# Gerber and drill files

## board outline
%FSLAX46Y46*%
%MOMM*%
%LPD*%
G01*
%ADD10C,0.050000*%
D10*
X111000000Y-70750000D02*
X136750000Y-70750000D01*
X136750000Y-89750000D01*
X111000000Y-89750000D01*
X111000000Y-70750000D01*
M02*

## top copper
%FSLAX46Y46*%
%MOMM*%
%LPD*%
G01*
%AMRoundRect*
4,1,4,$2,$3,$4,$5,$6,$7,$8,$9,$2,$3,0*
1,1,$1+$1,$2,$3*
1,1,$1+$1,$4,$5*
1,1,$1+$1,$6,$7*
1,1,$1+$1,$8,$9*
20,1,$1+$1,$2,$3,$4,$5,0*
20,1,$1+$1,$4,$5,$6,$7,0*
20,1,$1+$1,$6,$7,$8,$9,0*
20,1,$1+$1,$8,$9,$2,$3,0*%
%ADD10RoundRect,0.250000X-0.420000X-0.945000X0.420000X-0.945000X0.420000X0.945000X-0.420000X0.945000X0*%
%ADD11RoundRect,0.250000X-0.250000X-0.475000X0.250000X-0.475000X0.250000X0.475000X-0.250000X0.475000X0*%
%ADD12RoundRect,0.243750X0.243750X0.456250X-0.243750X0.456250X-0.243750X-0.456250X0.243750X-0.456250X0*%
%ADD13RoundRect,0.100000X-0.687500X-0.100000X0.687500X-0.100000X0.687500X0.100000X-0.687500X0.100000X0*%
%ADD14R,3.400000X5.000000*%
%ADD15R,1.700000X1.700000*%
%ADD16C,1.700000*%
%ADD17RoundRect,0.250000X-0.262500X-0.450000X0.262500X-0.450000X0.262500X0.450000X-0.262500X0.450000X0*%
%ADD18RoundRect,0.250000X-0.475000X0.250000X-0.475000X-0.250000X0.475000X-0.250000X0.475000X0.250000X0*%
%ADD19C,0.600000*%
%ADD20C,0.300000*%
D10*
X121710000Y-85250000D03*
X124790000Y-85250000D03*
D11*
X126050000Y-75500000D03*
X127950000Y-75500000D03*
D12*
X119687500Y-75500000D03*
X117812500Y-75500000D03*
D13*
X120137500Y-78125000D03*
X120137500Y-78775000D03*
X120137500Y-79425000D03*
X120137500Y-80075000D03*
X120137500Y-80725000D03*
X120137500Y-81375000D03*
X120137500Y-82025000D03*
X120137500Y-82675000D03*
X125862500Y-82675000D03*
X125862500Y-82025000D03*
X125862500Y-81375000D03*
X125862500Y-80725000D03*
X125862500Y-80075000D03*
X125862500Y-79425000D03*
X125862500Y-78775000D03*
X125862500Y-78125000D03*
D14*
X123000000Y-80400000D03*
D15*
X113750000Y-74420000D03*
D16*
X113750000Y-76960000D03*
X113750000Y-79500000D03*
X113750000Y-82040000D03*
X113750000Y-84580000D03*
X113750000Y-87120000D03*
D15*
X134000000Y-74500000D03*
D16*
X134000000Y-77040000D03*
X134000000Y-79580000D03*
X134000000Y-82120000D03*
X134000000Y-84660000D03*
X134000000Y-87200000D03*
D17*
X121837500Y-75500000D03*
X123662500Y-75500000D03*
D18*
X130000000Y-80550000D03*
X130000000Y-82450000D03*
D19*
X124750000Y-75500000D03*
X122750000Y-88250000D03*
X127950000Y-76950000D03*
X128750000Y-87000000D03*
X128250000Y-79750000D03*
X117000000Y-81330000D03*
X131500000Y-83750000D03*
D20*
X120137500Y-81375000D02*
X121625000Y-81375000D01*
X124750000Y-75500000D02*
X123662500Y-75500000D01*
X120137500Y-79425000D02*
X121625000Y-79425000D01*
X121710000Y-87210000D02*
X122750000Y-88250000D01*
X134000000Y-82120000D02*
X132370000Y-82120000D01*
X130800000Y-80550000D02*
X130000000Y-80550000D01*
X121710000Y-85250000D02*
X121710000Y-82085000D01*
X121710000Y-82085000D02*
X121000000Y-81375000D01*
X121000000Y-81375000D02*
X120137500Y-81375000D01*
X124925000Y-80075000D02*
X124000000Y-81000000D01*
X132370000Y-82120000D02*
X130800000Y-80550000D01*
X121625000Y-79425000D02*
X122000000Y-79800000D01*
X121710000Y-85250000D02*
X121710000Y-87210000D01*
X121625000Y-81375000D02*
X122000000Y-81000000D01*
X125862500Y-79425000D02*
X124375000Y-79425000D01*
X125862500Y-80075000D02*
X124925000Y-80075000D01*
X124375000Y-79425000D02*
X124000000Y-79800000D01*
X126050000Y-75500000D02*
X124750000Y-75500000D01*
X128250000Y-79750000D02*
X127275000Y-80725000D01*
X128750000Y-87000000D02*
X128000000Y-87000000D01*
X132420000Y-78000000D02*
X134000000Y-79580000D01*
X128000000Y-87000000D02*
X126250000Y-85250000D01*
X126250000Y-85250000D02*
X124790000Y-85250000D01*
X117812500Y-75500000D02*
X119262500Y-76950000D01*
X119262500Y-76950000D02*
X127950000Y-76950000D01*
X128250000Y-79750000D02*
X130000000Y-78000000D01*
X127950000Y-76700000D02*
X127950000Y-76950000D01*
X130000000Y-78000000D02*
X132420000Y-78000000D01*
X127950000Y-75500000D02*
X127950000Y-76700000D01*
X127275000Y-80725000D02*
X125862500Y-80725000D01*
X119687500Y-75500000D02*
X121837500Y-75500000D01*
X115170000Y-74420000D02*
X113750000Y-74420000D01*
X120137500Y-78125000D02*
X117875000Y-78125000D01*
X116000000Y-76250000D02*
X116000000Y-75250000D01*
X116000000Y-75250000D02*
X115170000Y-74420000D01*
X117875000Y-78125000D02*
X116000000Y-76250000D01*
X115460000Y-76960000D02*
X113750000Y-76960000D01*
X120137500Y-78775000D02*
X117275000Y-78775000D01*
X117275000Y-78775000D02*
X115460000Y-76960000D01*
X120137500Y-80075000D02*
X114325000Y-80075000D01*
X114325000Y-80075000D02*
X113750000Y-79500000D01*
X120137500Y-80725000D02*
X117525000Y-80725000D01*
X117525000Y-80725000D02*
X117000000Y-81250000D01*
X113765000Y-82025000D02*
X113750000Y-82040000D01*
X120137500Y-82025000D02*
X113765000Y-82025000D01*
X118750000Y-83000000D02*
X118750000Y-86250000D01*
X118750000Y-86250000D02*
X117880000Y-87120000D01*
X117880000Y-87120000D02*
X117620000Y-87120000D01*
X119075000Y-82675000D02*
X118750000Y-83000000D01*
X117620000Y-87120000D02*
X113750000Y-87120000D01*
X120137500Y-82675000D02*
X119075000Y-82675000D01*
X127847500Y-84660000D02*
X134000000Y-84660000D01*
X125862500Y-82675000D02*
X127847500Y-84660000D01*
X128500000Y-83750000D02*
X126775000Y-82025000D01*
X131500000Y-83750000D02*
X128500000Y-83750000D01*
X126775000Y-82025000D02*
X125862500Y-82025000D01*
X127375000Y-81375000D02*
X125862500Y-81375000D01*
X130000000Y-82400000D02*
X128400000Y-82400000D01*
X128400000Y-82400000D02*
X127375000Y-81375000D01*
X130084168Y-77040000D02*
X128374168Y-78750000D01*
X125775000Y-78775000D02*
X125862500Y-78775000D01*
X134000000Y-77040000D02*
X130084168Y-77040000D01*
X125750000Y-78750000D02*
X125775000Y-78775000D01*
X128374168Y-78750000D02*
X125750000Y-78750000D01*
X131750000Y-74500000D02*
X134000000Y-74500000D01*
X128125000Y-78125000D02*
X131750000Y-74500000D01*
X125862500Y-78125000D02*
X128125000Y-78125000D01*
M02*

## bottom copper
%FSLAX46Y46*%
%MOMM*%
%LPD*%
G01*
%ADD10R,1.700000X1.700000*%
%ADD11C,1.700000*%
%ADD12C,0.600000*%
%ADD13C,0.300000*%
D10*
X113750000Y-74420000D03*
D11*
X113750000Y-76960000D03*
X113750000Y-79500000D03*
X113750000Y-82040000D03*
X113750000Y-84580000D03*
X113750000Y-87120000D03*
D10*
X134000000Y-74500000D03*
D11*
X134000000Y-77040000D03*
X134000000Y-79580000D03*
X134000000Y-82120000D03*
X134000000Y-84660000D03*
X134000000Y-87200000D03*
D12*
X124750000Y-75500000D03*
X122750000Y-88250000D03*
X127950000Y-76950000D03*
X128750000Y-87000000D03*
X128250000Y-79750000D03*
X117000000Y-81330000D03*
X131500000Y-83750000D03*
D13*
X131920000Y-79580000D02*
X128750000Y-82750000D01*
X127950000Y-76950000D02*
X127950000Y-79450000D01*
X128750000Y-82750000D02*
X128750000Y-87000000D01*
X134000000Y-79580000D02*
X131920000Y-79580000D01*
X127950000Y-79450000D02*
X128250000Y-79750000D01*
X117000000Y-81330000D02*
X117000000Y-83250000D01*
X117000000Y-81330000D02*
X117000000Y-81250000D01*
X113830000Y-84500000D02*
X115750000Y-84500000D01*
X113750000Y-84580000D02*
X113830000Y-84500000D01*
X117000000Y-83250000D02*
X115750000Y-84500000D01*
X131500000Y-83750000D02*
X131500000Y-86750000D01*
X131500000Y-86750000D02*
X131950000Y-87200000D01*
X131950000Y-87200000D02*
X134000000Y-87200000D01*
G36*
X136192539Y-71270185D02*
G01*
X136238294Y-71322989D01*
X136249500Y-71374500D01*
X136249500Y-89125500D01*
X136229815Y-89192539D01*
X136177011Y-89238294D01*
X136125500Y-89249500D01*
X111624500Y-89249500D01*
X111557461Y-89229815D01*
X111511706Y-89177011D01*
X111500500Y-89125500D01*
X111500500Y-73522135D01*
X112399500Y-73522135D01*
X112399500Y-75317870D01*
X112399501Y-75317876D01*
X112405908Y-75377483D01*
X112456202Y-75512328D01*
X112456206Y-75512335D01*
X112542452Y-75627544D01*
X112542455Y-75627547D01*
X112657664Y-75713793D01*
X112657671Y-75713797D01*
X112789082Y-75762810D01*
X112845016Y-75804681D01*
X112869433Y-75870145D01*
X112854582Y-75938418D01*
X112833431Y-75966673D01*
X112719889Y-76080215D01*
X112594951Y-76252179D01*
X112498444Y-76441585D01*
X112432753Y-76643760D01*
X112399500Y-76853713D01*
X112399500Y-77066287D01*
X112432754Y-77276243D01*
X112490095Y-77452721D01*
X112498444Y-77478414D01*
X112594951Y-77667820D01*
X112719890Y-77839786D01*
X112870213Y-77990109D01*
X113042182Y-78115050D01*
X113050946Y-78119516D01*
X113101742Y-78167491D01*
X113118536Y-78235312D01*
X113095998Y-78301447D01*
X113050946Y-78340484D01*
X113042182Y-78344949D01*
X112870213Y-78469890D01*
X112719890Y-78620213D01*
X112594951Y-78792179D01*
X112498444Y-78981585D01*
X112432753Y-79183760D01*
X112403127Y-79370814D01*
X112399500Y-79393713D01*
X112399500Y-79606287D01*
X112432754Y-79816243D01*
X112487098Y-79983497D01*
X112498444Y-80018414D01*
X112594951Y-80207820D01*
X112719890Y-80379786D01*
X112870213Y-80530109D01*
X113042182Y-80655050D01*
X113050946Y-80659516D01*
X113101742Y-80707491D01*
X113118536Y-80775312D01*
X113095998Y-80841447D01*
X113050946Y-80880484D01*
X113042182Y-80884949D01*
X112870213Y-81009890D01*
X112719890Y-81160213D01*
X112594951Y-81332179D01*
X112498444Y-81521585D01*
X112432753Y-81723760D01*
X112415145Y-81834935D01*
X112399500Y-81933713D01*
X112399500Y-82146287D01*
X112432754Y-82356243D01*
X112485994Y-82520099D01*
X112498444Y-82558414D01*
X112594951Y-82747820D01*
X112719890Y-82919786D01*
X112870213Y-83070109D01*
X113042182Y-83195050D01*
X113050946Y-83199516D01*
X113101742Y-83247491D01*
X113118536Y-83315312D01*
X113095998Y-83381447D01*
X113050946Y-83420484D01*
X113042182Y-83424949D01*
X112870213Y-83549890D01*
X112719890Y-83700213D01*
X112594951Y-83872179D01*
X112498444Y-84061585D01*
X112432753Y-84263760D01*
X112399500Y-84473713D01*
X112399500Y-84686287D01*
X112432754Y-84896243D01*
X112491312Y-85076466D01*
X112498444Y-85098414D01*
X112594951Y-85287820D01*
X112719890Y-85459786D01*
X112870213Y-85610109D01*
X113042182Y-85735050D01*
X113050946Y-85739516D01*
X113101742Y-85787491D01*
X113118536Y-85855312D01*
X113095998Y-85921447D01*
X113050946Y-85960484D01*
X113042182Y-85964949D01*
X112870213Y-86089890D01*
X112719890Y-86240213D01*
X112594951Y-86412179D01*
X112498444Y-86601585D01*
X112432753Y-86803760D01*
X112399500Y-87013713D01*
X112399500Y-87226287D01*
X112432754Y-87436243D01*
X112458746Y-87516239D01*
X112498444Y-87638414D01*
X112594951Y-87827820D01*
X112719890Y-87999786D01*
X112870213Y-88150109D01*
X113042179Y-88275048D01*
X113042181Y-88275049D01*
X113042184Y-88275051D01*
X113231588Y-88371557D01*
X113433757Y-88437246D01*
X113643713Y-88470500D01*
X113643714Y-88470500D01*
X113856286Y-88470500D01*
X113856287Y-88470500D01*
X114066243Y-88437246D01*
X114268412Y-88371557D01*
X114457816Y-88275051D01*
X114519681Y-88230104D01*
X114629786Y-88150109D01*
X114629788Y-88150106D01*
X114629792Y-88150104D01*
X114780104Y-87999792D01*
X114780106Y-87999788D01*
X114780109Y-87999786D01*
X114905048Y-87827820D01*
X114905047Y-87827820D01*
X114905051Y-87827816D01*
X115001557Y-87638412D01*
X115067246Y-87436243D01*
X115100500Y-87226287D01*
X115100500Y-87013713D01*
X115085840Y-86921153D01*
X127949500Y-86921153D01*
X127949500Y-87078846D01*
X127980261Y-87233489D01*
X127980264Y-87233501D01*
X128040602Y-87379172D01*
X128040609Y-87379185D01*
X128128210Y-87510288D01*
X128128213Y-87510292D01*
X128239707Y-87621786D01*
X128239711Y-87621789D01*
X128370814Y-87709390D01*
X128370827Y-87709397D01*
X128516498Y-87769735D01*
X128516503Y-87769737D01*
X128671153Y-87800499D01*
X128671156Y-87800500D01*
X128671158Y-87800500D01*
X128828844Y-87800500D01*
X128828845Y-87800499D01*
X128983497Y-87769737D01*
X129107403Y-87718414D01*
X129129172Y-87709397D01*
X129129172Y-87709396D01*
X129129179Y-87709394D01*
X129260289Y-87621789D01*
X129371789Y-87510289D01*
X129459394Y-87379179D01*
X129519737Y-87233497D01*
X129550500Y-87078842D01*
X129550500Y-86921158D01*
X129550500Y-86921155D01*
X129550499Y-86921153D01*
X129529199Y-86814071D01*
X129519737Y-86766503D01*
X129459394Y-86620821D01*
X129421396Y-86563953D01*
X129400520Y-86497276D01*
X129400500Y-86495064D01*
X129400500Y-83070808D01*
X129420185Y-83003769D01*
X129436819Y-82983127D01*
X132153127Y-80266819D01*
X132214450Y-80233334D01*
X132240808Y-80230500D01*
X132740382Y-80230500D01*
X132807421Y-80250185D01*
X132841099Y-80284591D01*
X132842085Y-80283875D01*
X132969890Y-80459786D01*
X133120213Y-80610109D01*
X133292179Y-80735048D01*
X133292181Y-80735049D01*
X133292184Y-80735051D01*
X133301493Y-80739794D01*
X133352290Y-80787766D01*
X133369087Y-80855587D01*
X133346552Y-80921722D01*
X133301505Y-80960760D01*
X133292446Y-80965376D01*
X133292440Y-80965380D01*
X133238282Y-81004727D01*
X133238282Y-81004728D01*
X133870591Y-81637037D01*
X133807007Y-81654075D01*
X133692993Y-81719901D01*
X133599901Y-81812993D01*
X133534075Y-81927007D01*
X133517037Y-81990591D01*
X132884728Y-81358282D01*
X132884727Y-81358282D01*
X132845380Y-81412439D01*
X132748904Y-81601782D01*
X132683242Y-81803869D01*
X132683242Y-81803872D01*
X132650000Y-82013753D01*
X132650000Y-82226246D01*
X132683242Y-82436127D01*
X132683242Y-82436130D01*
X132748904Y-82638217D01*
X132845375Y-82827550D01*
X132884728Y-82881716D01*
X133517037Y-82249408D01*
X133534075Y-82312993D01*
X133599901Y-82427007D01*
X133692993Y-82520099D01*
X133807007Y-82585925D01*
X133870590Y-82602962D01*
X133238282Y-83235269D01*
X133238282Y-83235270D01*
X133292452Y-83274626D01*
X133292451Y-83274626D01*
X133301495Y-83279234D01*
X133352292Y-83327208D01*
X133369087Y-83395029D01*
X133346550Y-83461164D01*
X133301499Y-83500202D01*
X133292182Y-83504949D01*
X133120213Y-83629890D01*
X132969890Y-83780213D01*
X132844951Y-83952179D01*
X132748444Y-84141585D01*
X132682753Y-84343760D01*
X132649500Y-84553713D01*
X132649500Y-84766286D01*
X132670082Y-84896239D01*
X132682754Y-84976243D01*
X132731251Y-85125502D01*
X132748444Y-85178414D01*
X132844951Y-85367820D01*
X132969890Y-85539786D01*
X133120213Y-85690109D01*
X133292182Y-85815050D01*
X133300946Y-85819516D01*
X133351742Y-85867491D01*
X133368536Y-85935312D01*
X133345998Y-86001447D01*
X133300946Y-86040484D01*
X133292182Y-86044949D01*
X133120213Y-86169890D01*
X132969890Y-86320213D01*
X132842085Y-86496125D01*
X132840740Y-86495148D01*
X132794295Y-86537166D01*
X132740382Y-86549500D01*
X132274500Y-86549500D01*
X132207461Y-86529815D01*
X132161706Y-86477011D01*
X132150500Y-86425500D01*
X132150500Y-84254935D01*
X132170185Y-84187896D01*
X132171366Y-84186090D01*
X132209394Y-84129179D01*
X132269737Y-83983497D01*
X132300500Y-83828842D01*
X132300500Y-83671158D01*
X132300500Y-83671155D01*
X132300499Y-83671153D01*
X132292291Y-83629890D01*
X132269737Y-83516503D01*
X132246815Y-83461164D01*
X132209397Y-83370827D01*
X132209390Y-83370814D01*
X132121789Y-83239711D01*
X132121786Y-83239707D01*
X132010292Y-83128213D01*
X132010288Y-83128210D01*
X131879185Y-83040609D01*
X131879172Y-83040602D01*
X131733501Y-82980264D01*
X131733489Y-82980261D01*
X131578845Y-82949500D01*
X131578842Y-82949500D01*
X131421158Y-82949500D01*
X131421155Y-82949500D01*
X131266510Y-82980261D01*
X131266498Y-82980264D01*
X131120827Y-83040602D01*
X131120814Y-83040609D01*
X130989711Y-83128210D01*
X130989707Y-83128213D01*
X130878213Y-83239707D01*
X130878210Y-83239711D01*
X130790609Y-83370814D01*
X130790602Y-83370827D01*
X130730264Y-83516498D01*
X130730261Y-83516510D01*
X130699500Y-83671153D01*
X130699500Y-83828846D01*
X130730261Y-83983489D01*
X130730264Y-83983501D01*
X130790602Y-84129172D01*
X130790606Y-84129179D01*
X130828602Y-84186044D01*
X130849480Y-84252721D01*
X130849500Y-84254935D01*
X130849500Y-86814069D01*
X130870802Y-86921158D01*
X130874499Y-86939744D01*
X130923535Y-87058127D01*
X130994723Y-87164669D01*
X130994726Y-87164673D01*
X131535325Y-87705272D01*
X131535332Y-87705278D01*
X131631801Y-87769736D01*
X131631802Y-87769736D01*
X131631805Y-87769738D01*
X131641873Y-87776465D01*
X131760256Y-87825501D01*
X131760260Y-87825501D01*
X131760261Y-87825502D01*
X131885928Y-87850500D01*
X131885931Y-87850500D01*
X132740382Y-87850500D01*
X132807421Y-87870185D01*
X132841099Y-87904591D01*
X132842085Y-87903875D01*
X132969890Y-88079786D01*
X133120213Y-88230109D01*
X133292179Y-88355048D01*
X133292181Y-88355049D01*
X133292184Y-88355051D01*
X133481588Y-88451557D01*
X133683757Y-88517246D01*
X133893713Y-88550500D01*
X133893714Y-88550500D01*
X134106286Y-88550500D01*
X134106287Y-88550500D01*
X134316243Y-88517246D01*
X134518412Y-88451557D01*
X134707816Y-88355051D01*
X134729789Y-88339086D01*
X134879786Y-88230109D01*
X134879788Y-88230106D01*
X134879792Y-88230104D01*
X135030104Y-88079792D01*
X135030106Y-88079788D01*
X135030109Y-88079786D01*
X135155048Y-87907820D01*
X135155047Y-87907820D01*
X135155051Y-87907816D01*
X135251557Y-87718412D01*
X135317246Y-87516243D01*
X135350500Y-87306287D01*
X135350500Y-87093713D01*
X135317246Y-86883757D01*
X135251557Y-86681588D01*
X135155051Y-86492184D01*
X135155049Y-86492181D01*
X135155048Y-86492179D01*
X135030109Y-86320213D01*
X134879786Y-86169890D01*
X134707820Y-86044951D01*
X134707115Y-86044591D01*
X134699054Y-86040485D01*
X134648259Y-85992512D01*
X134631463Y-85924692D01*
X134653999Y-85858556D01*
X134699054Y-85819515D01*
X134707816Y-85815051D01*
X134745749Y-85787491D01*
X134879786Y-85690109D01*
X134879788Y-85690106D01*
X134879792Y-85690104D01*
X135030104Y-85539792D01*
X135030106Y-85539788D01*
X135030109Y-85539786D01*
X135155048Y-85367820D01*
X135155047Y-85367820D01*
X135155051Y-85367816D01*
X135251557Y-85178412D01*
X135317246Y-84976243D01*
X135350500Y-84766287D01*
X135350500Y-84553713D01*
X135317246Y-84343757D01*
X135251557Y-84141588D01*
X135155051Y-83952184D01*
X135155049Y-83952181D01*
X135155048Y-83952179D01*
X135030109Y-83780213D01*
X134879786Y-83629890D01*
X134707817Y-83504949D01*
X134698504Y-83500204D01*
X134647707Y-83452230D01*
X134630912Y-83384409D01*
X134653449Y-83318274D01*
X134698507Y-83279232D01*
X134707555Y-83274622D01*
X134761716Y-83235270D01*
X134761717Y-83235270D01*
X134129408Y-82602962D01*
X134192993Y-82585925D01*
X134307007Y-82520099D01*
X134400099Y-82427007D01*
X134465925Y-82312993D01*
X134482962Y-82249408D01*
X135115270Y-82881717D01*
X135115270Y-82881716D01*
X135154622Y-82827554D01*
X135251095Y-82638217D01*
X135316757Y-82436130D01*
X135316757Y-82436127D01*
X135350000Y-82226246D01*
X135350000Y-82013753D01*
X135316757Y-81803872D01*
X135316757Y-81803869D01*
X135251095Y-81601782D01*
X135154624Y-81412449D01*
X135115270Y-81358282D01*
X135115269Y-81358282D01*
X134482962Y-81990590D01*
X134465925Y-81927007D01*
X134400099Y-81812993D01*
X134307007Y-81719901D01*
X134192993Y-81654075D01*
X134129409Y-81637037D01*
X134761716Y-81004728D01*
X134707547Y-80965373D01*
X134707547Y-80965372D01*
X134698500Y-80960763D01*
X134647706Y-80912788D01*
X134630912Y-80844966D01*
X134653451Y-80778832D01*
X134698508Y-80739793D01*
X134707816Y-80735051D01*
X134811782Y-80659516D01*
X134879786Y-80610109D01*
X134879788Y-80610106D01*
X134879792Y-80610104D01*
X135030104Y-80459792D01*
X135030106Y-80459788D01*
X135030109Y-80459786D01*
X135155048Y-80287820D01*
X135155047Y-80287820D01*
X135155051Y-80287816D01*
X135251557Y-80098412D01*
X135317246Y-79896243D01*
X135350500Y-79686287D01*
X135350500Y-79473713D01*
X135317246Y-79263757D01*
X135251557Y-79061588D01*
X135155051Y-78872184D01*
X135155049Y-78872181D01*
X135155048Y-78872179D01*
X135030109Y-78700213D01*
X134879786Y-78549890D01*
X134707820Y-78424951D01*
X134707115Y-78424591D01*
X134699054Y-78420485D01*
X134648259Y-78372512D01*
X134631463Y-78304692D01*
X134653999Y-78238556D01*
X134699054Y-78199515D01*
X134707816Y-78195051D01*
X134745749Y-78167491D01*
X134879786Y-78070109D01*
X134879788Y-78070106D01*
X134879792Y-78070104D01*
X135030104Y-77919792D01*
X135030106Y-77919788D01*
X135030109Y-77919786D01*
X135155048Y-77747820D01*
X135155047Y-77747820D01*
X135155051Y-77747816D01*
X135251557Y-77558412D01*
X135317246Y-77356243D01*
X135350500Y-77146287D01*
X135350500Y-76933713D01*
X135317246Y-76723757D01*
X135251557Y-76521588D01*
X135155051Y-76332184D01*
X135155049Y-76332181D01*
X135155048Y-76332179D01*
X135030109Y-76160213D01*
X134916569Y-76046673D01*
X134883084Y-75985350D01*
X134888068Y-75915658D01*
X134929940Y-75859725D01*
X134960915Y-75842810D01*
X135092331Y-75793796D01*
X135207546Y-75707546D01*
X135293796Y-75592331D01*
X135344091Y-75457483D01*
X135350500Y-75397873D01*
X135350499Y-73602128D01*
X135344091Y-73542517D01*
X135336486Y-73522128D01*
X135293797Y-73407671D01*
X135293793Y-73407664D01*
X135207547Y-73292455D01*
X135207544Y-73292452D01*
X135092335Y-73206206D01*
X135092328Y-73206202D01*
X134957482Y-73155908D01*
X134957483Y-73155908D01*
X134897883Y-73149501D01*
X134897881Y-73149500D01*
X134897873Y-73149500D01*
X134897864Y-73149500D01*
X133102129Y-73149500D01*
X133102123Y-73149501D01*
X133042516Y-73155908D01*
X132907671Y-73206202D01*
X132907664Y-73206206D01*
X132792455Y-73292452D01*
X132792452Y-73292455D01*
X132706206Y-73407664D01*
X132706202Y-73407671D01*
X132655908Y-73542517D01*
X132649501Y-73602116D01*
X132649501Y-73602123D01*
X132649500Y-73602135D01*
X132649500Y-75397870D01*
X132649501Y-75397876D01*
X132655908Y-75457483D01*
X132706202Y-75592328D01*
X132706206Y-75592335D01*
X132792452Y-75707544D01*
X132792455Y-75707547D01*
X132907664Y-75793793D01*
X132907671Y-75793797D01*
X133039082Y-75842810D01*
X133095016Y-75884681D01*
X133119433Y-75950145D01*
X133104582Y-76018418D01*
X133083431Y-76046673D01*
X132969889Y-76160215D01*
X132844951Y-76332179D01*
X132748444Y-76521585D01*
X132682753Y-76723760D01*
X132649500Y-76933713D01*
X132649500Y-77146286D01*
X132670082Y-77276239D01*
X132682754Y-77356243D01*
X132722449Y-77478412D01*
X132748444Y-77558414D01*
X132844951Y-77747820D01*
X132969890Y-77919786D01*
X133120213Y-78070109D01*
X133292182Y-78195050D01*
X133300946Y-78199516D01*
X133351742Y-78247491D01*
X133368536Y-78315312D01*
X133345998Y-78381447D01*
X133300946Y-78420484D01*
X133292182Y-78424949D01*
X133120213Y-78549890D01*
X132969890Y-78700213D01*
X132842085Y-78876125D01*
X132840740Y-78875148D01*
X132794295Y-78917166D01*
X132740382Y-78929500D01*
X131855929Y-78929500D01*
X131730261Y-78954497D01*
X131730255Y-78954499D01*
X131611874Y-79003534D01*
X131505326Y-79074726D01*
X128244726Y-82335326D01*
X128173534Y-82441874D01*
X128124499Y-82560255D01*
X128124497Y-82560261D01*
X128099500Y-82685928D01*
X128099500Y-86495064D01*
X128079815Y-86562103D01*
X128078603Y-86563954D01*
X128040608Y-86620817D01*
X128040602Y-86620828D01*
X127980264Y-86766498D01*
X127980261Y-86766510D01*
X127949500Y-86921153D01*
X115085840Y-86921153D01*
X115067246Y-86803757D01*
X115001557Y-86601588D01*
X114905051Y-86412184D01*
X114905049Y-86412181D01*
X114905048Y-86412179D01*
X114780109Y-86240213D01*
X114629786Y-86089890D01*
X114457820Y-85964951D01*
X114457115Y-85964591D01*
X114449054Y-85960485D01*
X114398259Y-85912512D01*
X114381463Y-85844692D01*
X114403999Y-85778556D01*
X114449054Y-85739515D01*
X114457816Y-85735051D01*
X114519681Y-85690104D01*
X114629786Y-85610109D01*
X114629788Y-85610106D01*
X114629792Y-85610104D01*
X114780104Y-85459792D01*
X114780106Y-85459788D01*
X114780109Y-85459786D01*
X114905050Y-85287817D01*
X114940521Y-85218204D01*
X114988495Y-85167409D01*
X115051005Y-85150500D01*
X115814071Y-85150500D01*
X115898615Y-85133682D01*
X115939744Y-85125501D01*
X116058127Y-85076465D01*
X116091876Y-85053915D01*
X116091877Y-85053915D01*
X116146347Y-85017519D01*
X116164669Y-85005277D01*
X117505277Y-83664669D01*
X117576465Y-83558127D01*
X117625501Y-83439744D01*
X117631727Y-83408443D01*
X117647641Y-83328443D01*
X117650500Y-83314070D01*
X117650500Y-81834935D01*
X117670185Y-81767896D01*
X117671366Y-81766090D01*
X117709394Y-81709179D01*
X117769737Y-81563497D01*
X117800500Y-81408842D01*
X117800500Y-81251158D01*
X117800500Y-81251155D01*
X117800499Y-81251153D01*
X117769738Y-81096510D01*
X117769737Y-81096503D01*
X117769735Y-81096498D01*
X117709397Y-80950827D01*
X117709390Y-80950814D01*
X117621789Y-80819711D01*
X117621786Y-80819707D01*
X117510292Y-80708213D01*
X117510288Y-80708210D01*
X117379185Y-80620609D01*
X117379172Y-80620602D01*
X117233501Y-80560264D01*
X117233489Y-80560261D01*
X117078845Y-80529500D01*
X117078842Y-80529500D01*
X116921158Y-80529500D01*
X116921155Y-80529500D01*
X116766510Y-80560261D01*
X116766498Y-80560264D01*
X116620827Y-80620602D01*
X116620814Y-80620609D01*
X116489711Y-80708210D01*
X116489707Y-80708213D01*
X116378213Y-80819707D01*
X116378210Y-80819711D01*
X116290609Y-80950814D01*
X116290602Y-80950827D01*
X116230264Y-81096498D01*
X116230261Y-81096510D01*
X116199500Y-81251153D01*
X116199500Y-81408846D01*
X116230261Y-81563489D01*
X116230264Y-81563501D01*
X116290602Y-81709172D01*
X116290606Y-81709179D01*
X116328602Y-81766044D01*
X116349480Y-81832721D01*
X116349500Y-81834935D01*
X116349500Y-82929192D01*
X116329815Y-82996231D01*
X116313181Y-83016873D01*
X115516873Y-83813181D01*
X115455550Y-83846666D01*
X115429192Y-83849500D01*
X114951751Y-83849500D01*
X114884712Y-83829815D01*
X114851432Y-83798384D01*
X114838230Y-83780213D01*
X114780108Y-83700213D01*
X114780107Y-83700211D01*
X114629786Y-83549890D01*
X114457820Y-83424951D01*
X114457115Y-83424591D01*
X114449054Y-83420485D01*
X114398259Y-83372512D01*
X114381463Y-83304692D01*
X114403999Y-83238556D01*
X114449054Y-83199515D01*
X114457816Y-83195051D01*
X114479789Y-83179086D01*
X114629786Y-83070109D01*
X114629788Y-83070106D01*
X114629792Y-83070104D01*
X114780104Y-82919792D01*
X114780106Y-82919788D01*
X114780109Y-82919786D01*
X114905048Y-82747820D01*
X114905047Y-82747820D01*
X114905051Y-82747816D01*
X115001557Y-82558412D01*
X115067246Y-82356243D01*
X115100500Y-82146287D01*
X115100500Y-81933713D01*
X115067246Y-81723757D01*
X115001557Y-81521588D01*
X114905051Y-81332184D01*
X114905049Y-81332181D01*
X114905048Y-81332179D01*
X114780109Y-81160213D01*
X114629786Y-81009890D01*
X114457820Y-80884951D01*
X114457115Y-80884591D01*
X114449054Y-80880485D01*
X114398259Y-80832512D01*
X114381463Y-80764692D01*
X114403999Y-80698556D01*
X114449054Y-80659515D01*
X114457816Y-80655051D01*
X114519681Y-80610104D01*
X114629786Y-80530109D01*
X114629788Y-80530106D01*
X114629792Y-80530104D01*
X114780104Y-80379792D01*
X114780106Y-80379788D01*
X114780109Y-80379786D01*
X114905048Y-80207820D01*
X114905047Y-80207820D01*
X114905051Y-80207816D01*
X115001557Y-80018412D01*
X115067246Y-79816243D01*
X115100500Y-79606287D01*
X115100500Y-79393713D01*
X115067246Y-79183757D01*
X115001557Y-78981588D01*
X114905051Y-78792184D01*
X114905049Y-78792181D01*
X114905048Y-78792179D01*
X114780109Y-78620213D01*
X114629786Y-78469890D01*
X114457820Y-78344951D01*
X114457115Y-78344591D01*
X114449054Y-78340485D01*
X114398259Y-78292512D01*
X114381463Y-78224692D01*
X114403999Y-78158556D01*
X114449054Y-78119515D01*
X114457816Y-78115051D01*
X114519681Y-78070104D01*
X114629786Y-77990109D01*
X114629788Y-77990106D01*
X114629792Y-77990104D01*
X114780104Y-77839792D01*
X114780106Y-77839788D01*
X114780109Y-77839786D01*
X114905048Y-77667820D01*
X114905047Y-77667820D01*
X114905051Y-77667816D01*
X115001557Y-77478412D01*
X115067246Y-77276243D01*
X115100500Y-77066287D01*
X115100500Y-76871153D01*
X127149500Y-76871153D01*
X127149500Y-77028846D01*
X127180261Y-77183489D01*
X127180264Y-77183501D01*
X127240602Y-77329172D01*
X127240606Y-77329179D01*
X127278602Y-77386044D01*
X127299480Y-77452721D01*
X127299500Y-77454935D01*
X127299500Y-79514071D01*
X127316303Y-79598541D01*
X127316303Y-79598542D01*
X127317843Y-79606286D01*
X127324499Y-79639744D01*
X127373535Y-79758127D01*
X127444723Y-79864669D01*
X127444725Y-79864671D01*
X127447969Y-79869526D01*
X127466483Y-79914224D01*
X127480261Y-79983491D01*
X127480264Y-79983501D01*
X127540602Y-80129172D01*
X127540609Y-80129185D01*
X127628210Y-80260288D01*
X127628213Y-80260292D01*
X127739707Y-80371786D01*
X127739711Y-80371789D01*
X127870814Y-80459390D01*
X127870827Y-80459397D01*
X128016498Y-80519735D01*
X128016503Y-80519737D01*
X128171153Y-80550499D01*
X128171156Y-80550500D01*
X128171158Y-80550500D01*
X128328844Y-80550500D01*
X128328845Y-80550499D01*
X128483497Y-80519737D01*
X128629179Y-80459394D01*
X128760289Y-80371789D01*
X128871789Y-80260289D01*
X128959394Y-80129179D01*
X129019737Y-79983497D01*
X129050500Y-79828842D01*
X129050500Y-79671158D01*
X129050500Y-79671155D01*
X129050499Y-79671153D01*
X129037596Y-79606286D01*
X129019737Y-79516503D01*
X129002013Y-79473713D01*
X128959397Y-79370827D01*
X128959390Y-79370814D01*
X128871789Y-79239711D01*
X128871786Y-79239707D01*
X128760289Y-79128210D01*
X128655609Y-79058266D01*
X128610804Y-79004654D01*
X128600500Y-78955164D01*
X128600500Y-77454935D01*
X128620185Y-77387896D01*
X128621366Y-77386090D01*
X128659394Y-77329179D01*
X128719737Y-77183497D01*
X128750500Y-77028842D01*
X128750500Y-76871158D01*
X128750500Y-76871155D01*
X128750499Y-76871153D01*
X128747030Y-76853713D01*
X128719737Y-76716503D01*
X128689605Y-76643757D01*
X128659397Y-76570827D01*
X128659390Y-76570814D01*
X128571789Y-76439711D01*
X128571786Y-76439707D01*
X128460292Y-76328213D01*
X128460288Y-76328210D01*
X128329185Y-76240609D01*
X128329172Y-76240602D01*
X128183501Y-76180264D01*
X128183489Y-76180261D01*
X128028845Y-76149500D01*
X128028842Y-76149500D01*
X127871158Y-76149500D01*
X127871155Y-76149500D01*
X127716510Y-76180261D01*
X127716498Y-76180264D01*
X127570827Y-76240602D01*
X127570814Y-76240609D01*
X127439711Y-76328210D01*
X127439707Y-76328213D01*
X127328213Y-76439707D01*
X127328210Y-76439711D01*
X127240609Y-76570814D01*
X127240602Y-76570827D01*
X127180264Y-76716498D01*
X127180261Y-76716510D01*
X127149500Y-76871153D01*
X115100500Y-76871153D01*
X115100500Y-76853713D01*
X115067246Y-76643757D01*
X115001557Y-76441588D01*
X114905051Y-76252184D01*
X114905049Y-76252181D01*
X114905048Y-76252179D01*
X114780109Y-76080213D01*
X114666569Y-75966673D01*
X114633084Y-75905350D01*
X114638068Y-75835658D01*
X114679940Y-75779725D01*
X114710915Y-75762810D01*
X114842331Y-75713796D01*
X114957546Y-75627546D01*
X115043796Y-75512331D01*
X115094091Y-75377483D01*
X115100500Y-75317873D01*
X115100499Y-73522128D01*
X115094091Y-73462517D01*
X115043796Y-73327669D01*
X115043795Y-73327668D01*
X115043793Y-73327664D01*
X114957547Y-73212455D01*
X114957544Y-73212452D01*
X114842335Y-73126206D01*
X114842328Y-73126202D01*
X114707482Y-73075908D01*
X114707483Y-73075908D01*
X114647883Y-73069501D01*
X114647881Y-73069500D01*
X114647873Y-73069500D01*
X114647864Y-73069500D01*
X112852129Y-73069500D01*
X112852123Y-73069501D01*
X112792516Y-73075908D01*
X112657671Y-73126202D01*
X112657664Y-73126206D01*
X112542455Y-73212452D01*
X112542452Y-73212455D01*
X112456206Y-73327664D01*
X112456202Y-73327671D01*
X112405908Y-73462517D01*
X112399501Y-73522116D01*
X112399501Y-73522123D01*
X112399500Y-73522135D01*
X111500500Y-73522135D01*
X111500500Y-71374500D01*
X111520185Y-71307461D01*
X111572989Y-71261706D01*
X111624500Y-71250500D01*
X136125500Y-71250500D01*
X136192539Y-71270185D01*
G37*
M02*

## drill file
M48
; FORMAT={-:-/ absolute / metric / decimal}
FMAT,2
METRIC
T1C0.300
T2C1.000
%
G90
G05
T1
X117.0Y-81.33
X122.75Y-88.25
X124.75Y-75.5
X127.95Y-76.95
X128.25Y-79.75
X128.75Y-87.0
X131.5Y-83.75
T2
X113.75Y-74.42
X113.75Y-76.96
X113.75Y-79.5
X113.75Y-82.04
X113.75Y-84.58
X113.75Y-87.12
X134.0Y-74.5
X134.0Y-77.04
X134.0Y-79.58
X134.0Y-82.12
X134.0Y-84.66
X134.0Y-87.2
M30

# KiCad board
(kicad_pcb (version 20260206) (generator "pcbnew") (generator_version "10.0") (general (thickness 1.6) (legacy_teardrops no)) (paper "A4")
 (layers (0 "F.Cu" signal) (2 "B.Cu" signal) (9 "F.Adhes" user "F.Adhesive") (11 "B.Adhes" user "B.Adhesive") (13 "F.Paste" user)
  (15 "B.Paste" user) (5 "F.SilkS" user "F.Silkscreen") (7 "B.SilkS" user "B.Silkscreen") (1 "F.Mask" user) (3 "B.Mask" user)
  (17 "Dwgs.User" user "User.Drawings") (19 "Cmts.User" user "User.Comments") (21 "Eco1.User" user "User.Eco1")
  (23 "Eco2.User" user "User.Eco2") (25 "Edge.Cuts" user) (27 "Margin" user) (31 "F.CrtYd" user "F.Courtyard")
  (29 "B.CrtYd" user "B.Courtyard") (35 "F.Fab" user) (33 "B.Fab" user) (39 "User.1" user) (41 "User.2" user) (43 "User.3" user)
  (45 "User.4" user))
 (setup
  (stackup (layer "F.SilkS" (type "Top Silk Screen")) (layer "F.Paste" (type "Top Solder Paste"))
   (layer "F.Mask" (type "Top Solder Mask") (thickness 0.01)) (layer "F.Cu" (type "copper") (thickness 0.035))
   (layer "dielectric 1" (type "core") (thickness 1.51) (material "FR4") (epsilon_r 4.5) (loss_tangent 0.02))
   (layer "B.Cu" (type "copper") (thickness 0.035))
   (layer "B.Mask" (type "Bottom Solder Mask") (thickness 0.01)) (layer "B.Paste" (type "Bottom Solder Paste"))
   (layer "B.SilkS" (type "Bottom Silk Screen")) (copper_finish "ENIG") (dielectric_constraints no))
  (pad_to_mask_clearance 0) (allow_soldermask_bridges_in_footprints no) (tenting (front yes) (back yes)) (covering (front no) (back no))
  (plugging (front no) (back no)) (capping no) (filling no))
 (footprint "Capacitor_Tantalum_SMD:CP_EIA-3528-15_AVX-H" (layer "F.Cu") (at 123.25 85.25)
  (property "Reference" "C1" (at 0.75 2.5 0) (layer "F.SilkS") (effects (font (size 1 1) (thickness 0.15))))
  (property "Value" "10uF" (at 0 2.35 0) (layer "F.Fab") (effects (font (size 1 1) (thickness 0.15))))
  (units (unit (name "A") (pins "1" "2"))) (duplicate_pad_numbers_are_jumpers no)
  (pad "1" smd roundrect (at -1.54 0) (size 1.34 2.39) (layers "F.Cu" "F.Mask" "F.Paste") (roundrect_rratio 0.186567) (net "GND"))
  (pad "2" smd roundrect (at 1.54 0) (size 1.34 2.39) (layers "F.Cu" "F.Mask" "F.Paste") (roundrect_rratio 0.186567) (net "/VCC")))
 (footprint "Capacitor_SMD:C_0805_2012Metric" (layer "F.Cu") (at 127 75.5)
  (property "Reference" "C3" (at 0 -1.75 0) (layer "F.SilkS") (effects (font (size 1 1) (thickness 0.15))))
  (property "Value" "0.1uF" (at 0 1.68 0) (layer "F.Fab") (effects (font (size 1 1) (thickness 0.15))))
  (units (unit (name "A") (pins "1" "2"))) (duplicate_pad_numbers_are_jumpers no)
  (pad "1" smd roundrect (at -0.95 0) (size 1 1.45) (layers "F.Cu" "F.Mask" "F.Paste") (roundrect_rratio 0.25) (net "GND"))
  (pad "2" smd roundrect (at 0.95 0) (size 1 1.45) (layers "F.Cu" "F.Mask" "F.Paste") (roundrect_rratio 0.25) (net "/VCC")))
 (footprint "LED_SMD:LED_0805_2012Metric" (layer "F.Cu") (at 118.75 75.5 180)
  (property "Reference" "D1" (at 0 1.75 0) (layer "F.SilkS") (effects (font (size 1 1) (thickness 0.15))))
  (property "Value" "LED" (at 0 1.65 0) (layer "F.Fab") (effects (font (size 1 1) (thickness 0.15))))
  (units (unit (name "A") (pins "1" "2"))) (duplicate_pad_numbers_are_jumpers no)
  (pad "1" smd roundrect (at -0.9375 0 180) (size 0.975 1.4) (layers "F.Cu" "F.Mask" "F.Paste") (roundrect_rratio 0.25) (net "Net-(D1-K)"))
  (pad "2" smd roundrect (at 0.9375 0 180) (size 0.975 1.4) (layers "F.Cu" "F.Mask" "F.Paste") (roundrect_rratio 0.25) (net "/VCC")))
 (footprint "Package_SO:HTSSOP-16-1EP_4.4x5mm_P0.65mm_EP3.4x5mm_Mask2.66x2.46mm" (layer "F.Cu") (at 123 80.4)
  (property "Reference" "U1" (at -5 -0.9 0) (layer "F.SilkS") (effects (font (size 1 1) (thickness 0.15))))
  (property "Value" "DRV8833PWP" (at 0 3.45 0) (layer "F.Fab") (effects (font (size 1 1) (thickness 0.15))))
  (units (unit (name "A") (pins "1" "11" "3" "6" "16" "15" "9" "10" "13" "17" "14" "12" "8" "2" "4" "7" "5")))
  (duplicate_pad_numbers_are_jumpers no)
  (pad "" smd roundrect (at 0 -0.615) (size 2.14 0.99) (layers "F.Paste") (roundrect_rratio 0.25))
  (pad "" smd rect (at 0 0) (size 2.66 2.46) (layers "F.Mask"))
  (pad "" smd roundrect (at 0 0.615) (size 2.14 0.99) (layers "F.Paste") (roundrect_rratio 0.25))
  (pad "1" smd roundrect (at -2.8625 -2.275) (size 1.575 0.4) (layers "F.Cu" "F.Mask" "F.Paste") (roundrect_rratio 0.25) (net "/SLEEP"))
  (pad "2" smd roundrect (at -2.8625 -1.625) (size 1.575 0.4) (layers "F.Cu" "F.Mask" "F.Paste") (roundrect_rratio 0.25) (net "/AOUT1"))
  (pad "3" smd roundrect (at -2.8625 -0.975) (size 1.575 0.4) (layers "F.Cu" "F.Mask" "F.Paste") (roundrect_rratio 0.25) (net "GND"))
  (pad "4" smd roundrect (at -2.8625 -0.325) (size 1.575 0.4) (layers "F.Cu" "F.Mask" "F.Paste") (roundrect_rratio 0.25) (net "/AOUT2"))
  (pad "5" smd roundrect (at -2.8625 0.325) (size 1.575 0.4) (layers "F.Cu" "F.Mask" "F.Paste") (roundrect_rratio 0.25) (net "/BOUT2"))
  (pad "6" smd roundrect (at -2.8625 0.975) (size 1.575 0.4) (layers "F.Cu" "F.Mask" "F.Paste") (roundrect_rratio 0.25) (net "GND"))
  (pad "7" smd roundrect (at -2.8625 1.625) (size 1.575 0.4) (layers "F.Cu" "F.Mask" "F.Paste") (roundrect_rratio 0.25) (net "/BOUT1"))
  (pad "8" smd roundrect (at -2.8625 2.275) (size 1.575 0.4) (layers "F.Cu" "F.Mask" "F.Paste") (roundrect_rratio 0.25) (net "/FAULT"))
  (pad "9" smd roundrect (at 2.8625 2.275) (size 1.575 0.4) (layers "F.Cu" "F.Mask" "F.Paste") (roundrect_rratio 0.25) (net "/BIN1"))
  (pad "10" smd roundrect (at 2.8625 1.625) (size 1.575 0.4) (layers "F.Cu" "F.Mask" "F.Paste") (roundrect_rratio 0.25) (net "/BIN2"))
  (pad "11" smd roundrect (at 2.8625 0.975) (size 1.575 0.4) (layers "F.Cu" "F.Mask" "F.Paste") (roundrect_rratio 0.25) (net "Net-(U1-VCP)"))
  (pad "12" smd roundrect (at 2.8625 0.325) (size 1.575 0.4) (layers "F.Cu" "F.Mask" "F.Paste") (roundrect_rratio 0.25) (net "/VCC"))
  (pad "13" smd roundrect (at 2.8625 -0.325) (size 1.575 0.4) (layers "F.Cu" "F.Mask" "F.Paste") (roundrect_rratio 0.25) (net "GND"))
  (pad "14" smd roundrect (at 2.8625 -0.975) (size 1.575 0.4) (layers "F.Cu" "F.Mask" "F.Paste") (roundrect_rratio 0.25) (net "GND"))
  (pad "15" smd roundrect (at 2.8625 -1.625) (size 1.575 0.4) (layers "F.Cu" "F.Mask" "F.Paste") (roundrect_rratio 0.25) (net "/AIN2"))
  (pad "16" smd roundrect (at 2.8625 -2.275) (size 1.575 0.4) (layers "F.Cu" "F.Mask" "F.Paste") (roundrect_rratio 0.25) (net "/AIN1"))
  (pad "17" smd rect (at 0 0) (size 3.4 5) (layers "F.Cu") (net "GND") (zone_connect 2)))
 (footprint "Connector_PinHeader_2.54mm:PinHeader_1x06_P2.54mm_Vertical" (layer "F.Cu") (at 113.75 74.42)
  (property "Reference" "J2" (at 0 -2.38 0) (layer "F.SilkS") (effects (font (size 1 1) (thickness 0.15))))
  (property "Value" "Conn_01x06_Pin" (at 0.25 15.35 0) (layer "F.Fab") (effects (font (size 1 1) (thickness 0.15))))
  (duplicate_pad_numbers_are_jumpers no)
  (pad "1" thru_hole rect (at 0 0) (size 1.7 1.7) (drill 1) (layers "*.Cu" "*.Mask") (remove_unused_layers no) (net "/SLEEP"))
  (pad "2" thru_hole circle (at 0 2.54) (size 1.7 1.7) (drill 1) (layers "*.Cu" "*.Mask") (remove_unused_layers no) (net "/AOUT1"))
  (pad "3" thru_hole circle (at 0 5.08) (size 1.7 1.7) (drill 1) (layers "*.Cu" "*.Mask") (remove_unused_layers no) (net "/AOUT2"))
  (pad "4" thru_hole circle (at 0 7.62) (size 1.7 1.7) (drill 1) (layers "*.Cu" "*.Mask") (remove_unused_layers no) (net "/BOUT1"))
  (pad "5" thru_hole circle (at 0 10.16) (size 1.7 1.7) (drill 1) (layers "*.Cu" "*.Mask") (remove_unused_layers no) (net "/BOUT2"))
  (pad "6" thru_hole circle (at 0 12.7) (size 1.7 1.7) (drill 1) (layers "*.Cu" "*.Mask") (remove_unused_layers no) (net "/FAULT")))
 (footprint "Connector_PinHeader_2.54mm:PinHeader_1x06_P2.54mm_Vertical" (layer "F.Cu") (at 134 74.5)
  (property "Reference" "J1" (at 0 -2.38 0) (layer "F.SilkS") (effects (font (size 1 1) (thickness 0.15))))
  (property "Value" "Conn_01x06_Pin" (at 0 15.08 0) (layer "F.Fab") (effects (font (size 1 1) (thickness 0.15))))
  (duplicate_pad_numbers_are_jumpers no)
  (pad "1" thru_hole rect (at 0 0) (size 1.7 1.7) (drill 1) (layers "*.Cu" "*.Mask") (remove_unused_layers no) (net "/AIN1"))
  (pad "2" thru_hole circle (at 0 2.54) (size 1.7 1.7) (drill 1) (layers "*.Cu" "*.Mask") (remove_unused_layers no) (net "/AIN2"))
  (pad "3" thru_hole circle (at 0 5.08) (size 1.7 1.7) (drill 1) (layers "*.Cu" "*.Mask") (remove_unused_layers no) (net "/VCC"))
  (pad "4" thru_hole circle (at 0 7.62) (size 1.7 1.7) (drill 1) (layers "*.Cu" "*.Mask") (remove_unused_layers no) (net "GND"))
  (pad "5" thru_hole circle (at 0 10.16) (size 1.7 1.7) (drill 1) (layers "*.Cu" "*.Mask") (remove_unused_layers no) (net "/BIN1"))
  (pad "6" thru_hole circle (at 0 12.7) (size 1.7 1.7) (drill 1) (layers "*.Cu" "*.Mask") (remove_unused_layers no) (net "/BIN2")))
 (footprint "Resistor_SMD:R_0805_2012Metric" (layer "F.Cu") (at 122.75 75.5)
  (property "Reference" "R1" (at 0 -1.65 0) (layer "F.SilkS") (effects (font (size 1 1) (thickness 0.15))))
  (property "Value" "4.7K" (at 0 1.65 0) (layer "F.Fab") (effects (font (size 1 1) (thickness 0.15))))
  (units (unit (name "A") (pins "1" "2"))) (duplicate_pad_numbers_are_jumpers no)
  (pad "1" smd roundrect (at -0.9125 0) (size 1.025 1.4) (layers "F.Cu" "F.Mask" "F.Paste") (roundrect_rratio 0.243902) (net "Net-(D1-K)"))
  (pad "2" smd roundrect (at 0.9125 0) (size 1.025 1.4) (layers "F.Cu" "F.Mask" "F.Paste") (roundrect_rratio 0.243902) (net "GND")))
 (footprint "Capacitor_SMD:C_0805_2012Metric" (layer "F.Cu") (at 130 81.5 -90)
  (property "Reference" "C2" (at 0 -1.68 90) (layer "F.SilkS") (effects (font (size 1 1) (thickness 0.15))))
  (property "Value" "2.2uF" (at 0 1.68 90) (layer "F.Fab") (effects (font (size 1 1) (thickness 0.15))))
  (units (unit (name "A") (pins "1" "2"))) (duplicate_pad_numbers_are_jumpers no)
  (pad "1" smd roundrect (at -0.95 0 270) (size 1 1.45) (layers "F.Cu" "F.Mask" "F.Paste") (roundrect_rratio 0.25) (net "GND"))
  (pad "2" smd roundrect (at 0.95 0 270) (size 1 1.45) (layers "F.Cu" "F.Mask" "F.Paste") (roundrect_rratio 0.25) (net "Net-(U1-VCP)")))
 (gr_rect (start 111 70.75) (end 136.75 89.75) (stroke (width 0.05) (type default)) (fill no) (layer "Edge.Cuts"))
 (segment (start 120.1375 81.375) (end 121.625 81.375) (width 0.3) (layer "F.Cu") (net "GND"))
 (segment (start 124.75 75.5) (end 123.6625 75.5) (width 0.3) (layer "F.Cu") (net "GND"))
 (segment (start 120.1375 79.425) (end 121.625 79.425) (width 0.3) (layer "F.Cu") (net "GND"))
 (segment (start 121.71 87.21) (end 122.75 88.25) (width 0.3) (layer "F.Cu") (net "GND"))
 (segment (start 134 82.12) (end 132.37 82.12) (width 0.3) (layer "F.Cu") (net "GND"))
 (segment (start 130.8 80.55) (end 130 80.55) (width 0.3) (layer "F.Cu") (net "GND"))
 (segment (start 121.71 85.25) (end 121.71 82.085) (width 0.3) (layer "F.Cu") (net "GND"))
 (segment (start 121.71 82.085) (end 121 81.375) (width 0.3) (layer "F.Cu") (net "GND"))
 (segment (start 121 81.375) (end 120.1375 81.375) (width 0.3) (layer "F.Cu") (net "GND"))
 (segment (start 124.925 80.075) (end 124 81) (width 0.3) (layer "F.Cu") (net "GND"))
 (segment (start 132.37 82.12) (end 130.8 80.55) (width 0.3) (layer "F.Cu") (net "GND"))
 (segment (start 121.625 79.425) (end 122 79.8) (width 0.3) (layer "F.Cu") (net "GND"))
 (segment (start 121.71 85.25) (end 121.71 87.21) (width 0.3) (layer "F.Cu") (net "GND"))
 (segment (start 121.625 81.375) (end 122 81) (width 0.3) (layer "F.Cu") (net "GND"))
 (segment (start 125.8625 79.425) (end 124.375 79.425) (width 0.3) (layer "F.Cu") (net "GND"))
 (segment (start 125.8625 80.075) (end 124.925 80.075) (width 0.3) (layer "F.Cu") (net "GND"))
 (segment (start 124.375 79.425) (end 124 79.8) (width 0.3) (layer "F.Cu") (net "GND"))
 (segment (start 126.05 75.5) (end 124.75 75.5) (width 0.3) (layer "F.Cu") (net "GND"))
 (via (at 124.75 75.5) (size 0.6) (drill 0.3) (layers "F.Cu" "B.Cu") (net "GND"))
 (via (at 122.75 88.25) (size 0.6) (drill 0.3) (layers "F.Cu" "B.Cu") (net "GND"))
 (segment (start 128.25 79.75) (end 127.275 80.725) (width 0.3) (layer "F.Cu") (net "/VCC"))
 (segment (start 128.75 87) (end 128 87) (width 0.3) (layer "F.Cu") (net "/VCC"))
 (segment (start 132.42 78) (end 134 79.58) (width 0.3) (layer "F.Cu") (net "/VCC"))
 (segment (start 128 87) (end 126.25 85.25) (width 0.3) (layer "F.Cu") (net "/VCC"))
 (segment (start 126.25 85.25) (end 124.79 85.25) (width 0.3) (layer "F.Cu") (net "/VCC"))
 (segment (start 117.8125 75.5) (end 119.2625 76.95) (width 0.3) (layer "F.Cu") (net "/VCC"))
 (segment (start 119.2625 76.95) (end 127.95 76.95) (width 0.3) (layer "F.Cu") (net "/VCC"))
 (segment (start 128.25 79.75) (end 130 78) (width 0.3) (layer "F.Cu") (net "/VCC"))
 (segment (start 127.95 76.7) (end 127.95 76.95) (width 0.3) (layer "F.Cu") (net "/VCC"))
 (segment (start 130 78) (end 132.42 78) (width 0.3) (layer "F.Cu") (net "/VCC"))
 (segment (start 127.95 75.5) (end 127.95 76.7) (width 0.3) (layer "F.Cu") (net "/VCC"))
 (segment (start 127.275 80.725) (end 125.8625 80.725) (width 0.3) (layer "F.Cu") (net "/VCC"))
 (via (at 127.95 76.95) (size 0.6) (drill 0.3) (layers "F.Cu" "B.Cu") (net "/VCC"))
 (via (at 128.75 87) (size 0.6) (drill 0.3) (layers "F.Cu" "B.Cu") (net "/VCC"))
 (via (at 128.25 79.75) (size 0.6) (drill 0.3) (layers "F.Cu" "B.Cu") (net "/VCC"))
 (segment (start 131.92 79.58) (end 128.75 82.75) (width 0.3) (layer "B.Cu") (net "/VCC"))
 (segment (start 127.95 76.95) (end 127.95 79.45) (width 0.3) (layer "B.Cu") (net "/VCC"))
 (segment (start 128.75 82.75) (end 128.75 87) (width 0.3) (layer "B.Cu") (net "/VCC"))
 (segment (start 134 79.58) (end 131.92 79.58) (width 0.3) (layer "B.Cu") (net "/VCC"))
 (segment (start 127.95 79.45) (end 128.25 79.75) (width 0.3) (layer "B.Cu") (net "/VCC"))
 (segment (start 119.6875 75.5) (end 121.8375 75.5) (width 0.3) (layer "F.Cu") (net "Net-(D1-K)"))
 (segment (start 115.17 74.42) (end 113.75 74.42) (width 0.3) (layer "F.Cu") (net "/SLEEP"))
 (segment (start 120.1375 78.125) (end 117.875 78.125) (width 0.3) (layer "F.Cu") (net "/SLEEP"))
 (segment (start 116 76.25) (end 116 75.25) (width 0.3) (layer "F.Cu") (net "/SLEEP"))
 (segment (start 116 75.25) (end 115.17 74.42) (width 0.3) (layer "F.Cu") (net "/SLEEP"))
 (segment (start 117.875 78.125) (end 116 76.25) (width 0.3) (layer "F.Cu") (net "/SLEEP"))
 (segment (start 115.46 76.96) (end 113.75 76.96) (width 0.3) (layer "F.Cu") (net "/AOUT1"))
 (segment (start 120.1375 78.775) (end 117.275 78.775) (width 0.3) (layer "F.Cu") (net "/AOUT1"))
 (segment (start 117.275 78.775) (end 115.46 76.96) (width 0.3) (layer "F.Cu") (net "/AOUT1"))
 (segment (start 120.1375 80.075) (end 114.325 80.075) (width 0.3) (layer "F.Cu") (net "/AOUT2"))
 (segment (start 114.325 80.075) (end 113.75 79.5) (width 0.3) (layer "F.Cu") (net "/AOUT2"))
 (segment (start 120.1375 80.725) (end 117.525 80.725) (width 0.3) (layer "F.Cu") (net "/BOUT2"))
 (segment (start 117.525 80.725) (end 117 81.25) (width 0.3) (layer "F.Cu") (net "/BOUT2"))
 (via (at 117 81.33) (size 0.6) (drill 0.3) (layers "F.Cu" "B.Cu") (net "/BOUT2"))
 (segment (start 117 81.33) (end 117 83.25) (width 0.3) (layer "B.Cu") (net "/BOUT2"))
 (segment (start 117 81.33) (end 117 81.25) (width 0.3) (layer "B.Cu") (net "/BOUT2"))
 (segment (start 113.83 84.5) (end 115.75 84.5) (width 0.3) (layer "B.Cu") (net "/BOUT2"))
 (segment (start 113.75 84.58) (end 113.83 84.5) (width 0.3) (layer "B.Cu") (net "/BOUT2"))
 (segment (start 117 83.25) (end 115.75 84.5) (width 0.3) (layer "B.Cu") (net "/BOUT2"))
 (segment (start 113.765 82.025) (end 113.75 82.04) (width 0.3) (layer "F.Cu") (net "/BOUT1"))
 (segment (start 120.1375 82.025) (end 113.765 82.025) (width 0.3) (layer "F.Cu") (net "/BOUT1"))
 (segment (start 118.75 83) (end 118.75 86.25) (width 0.3) (layer "F.Cu") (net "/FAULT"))
 (segment (start 118.75 86.25) (end 117.88 87.12) (width 0.3) (layer "F.Cu") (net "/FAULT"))
 (segment (start 117.88 87.12) (end 117.62 87.12) (width 0.3) (layer "F.Cu") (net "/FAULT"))
 (segment (start 119.075 82.675) (end 118.75 83) (width 0.3) (layer "F.Cu") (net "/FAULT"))
 (segment (start 117.62 87.12) (end 113.75 87.12) (width 0.3) (layer "F.Cu") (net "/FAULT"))
 (segment (start 120.1375 82.675) (end 119.075 82.675) (width 0.3) (layer "F.Cu") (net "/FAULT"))
 (segment (start 127.8475 84.66) (end 134 84.66) (width 0.3) (layer "F.Cu") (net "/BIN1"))
 (segment (start 125.8625 82.675) (end 127.8475 84.66) (width 0.3) (layer "F.Cu") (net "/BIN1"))
 (segment (start 128.5 83.75) (end 126.775 82.025) (width 0.3) (layer "F.Cu") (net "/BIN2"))
 (segment (start 131.5 83.75) (end 128.5 83.75) (width 0.3) (layer "F.Cu") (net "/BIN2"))
 (segment (start 126.775 82.025) (end 125.8625 82.025) (width 0.3) (layer "F.Cu") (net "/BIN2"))
 (via (at 131.5 83.75) (size 0.6) (drill 0.3) (layers "F.Cu" "B.Cu") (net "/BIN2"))
 (segment (start 131.5 83.75) (end 131.5 86.75) (width 0.3) (layer "B.Cu") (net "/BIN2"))
 (segment (start 131.5 86.75) (end 131.95 87.2) (width 0.3) (layer "B.Cu") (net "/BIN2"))
 (segment (start 131.95 87.2) (end 134 87.2) (width 0.3) (layer "B.Cu") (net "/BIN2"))
 (segment (start 127.375 81.375) (end 125.8625 81.375) (width 0.3) (layer "F.Cu") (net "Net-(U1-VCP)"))
 (segment (start 130 82.4) (end 128.4 82.4) (width 0.3) (layer "F.Cu") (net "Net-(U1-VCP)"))
 (segment (start 128.4 82.4) (end 127.375 81.375) (width 0.3) (layer "F.Cu") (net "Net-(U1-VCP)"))
 (segment (start 130.084168 77.04) (end 128.374168 78.75) (width 0.3) (layer "F.Cu") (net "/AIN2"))
 (segment (start 125.775 78.775) (end 125.8625 78.775) (width 0.3) (layer "F.Cu") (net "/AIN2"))
 (segment (start 134 77.04) (end 130.084168 77.04) (width 0.3) (layer "F.Cu") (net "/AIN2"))
 (segment (start 125.75 78.75) (end 125.775 78.775) (width 0.3) (layer "F.Cu") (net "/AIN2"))
 (segment (start 128.374168 78.75) (end 125.75 78.75) (width 0.3) (layer "F.Cu") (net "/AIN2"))
 (segment (start 131.75 74.5) (end 134 74.5) (width 0.3) (layer "F.Cu") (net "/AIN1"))
 (segment (start 128.125 78.125) (end 131.75 74.5) (width 0.3) (layer "F.Cu") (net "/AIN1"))
 (segment (start 125.8625 78.125) (end 128.125 78.125) (width 0.3) (layer "F.Cu") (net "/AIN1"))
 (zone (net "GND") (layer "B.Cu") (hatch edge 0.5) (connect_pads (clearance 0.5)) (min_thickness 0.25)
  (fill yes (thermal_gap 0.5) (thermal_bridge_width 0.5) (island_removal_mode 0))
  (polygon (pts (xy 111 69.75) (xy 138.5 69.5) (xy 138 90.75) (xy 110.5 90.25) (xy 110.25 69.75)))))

